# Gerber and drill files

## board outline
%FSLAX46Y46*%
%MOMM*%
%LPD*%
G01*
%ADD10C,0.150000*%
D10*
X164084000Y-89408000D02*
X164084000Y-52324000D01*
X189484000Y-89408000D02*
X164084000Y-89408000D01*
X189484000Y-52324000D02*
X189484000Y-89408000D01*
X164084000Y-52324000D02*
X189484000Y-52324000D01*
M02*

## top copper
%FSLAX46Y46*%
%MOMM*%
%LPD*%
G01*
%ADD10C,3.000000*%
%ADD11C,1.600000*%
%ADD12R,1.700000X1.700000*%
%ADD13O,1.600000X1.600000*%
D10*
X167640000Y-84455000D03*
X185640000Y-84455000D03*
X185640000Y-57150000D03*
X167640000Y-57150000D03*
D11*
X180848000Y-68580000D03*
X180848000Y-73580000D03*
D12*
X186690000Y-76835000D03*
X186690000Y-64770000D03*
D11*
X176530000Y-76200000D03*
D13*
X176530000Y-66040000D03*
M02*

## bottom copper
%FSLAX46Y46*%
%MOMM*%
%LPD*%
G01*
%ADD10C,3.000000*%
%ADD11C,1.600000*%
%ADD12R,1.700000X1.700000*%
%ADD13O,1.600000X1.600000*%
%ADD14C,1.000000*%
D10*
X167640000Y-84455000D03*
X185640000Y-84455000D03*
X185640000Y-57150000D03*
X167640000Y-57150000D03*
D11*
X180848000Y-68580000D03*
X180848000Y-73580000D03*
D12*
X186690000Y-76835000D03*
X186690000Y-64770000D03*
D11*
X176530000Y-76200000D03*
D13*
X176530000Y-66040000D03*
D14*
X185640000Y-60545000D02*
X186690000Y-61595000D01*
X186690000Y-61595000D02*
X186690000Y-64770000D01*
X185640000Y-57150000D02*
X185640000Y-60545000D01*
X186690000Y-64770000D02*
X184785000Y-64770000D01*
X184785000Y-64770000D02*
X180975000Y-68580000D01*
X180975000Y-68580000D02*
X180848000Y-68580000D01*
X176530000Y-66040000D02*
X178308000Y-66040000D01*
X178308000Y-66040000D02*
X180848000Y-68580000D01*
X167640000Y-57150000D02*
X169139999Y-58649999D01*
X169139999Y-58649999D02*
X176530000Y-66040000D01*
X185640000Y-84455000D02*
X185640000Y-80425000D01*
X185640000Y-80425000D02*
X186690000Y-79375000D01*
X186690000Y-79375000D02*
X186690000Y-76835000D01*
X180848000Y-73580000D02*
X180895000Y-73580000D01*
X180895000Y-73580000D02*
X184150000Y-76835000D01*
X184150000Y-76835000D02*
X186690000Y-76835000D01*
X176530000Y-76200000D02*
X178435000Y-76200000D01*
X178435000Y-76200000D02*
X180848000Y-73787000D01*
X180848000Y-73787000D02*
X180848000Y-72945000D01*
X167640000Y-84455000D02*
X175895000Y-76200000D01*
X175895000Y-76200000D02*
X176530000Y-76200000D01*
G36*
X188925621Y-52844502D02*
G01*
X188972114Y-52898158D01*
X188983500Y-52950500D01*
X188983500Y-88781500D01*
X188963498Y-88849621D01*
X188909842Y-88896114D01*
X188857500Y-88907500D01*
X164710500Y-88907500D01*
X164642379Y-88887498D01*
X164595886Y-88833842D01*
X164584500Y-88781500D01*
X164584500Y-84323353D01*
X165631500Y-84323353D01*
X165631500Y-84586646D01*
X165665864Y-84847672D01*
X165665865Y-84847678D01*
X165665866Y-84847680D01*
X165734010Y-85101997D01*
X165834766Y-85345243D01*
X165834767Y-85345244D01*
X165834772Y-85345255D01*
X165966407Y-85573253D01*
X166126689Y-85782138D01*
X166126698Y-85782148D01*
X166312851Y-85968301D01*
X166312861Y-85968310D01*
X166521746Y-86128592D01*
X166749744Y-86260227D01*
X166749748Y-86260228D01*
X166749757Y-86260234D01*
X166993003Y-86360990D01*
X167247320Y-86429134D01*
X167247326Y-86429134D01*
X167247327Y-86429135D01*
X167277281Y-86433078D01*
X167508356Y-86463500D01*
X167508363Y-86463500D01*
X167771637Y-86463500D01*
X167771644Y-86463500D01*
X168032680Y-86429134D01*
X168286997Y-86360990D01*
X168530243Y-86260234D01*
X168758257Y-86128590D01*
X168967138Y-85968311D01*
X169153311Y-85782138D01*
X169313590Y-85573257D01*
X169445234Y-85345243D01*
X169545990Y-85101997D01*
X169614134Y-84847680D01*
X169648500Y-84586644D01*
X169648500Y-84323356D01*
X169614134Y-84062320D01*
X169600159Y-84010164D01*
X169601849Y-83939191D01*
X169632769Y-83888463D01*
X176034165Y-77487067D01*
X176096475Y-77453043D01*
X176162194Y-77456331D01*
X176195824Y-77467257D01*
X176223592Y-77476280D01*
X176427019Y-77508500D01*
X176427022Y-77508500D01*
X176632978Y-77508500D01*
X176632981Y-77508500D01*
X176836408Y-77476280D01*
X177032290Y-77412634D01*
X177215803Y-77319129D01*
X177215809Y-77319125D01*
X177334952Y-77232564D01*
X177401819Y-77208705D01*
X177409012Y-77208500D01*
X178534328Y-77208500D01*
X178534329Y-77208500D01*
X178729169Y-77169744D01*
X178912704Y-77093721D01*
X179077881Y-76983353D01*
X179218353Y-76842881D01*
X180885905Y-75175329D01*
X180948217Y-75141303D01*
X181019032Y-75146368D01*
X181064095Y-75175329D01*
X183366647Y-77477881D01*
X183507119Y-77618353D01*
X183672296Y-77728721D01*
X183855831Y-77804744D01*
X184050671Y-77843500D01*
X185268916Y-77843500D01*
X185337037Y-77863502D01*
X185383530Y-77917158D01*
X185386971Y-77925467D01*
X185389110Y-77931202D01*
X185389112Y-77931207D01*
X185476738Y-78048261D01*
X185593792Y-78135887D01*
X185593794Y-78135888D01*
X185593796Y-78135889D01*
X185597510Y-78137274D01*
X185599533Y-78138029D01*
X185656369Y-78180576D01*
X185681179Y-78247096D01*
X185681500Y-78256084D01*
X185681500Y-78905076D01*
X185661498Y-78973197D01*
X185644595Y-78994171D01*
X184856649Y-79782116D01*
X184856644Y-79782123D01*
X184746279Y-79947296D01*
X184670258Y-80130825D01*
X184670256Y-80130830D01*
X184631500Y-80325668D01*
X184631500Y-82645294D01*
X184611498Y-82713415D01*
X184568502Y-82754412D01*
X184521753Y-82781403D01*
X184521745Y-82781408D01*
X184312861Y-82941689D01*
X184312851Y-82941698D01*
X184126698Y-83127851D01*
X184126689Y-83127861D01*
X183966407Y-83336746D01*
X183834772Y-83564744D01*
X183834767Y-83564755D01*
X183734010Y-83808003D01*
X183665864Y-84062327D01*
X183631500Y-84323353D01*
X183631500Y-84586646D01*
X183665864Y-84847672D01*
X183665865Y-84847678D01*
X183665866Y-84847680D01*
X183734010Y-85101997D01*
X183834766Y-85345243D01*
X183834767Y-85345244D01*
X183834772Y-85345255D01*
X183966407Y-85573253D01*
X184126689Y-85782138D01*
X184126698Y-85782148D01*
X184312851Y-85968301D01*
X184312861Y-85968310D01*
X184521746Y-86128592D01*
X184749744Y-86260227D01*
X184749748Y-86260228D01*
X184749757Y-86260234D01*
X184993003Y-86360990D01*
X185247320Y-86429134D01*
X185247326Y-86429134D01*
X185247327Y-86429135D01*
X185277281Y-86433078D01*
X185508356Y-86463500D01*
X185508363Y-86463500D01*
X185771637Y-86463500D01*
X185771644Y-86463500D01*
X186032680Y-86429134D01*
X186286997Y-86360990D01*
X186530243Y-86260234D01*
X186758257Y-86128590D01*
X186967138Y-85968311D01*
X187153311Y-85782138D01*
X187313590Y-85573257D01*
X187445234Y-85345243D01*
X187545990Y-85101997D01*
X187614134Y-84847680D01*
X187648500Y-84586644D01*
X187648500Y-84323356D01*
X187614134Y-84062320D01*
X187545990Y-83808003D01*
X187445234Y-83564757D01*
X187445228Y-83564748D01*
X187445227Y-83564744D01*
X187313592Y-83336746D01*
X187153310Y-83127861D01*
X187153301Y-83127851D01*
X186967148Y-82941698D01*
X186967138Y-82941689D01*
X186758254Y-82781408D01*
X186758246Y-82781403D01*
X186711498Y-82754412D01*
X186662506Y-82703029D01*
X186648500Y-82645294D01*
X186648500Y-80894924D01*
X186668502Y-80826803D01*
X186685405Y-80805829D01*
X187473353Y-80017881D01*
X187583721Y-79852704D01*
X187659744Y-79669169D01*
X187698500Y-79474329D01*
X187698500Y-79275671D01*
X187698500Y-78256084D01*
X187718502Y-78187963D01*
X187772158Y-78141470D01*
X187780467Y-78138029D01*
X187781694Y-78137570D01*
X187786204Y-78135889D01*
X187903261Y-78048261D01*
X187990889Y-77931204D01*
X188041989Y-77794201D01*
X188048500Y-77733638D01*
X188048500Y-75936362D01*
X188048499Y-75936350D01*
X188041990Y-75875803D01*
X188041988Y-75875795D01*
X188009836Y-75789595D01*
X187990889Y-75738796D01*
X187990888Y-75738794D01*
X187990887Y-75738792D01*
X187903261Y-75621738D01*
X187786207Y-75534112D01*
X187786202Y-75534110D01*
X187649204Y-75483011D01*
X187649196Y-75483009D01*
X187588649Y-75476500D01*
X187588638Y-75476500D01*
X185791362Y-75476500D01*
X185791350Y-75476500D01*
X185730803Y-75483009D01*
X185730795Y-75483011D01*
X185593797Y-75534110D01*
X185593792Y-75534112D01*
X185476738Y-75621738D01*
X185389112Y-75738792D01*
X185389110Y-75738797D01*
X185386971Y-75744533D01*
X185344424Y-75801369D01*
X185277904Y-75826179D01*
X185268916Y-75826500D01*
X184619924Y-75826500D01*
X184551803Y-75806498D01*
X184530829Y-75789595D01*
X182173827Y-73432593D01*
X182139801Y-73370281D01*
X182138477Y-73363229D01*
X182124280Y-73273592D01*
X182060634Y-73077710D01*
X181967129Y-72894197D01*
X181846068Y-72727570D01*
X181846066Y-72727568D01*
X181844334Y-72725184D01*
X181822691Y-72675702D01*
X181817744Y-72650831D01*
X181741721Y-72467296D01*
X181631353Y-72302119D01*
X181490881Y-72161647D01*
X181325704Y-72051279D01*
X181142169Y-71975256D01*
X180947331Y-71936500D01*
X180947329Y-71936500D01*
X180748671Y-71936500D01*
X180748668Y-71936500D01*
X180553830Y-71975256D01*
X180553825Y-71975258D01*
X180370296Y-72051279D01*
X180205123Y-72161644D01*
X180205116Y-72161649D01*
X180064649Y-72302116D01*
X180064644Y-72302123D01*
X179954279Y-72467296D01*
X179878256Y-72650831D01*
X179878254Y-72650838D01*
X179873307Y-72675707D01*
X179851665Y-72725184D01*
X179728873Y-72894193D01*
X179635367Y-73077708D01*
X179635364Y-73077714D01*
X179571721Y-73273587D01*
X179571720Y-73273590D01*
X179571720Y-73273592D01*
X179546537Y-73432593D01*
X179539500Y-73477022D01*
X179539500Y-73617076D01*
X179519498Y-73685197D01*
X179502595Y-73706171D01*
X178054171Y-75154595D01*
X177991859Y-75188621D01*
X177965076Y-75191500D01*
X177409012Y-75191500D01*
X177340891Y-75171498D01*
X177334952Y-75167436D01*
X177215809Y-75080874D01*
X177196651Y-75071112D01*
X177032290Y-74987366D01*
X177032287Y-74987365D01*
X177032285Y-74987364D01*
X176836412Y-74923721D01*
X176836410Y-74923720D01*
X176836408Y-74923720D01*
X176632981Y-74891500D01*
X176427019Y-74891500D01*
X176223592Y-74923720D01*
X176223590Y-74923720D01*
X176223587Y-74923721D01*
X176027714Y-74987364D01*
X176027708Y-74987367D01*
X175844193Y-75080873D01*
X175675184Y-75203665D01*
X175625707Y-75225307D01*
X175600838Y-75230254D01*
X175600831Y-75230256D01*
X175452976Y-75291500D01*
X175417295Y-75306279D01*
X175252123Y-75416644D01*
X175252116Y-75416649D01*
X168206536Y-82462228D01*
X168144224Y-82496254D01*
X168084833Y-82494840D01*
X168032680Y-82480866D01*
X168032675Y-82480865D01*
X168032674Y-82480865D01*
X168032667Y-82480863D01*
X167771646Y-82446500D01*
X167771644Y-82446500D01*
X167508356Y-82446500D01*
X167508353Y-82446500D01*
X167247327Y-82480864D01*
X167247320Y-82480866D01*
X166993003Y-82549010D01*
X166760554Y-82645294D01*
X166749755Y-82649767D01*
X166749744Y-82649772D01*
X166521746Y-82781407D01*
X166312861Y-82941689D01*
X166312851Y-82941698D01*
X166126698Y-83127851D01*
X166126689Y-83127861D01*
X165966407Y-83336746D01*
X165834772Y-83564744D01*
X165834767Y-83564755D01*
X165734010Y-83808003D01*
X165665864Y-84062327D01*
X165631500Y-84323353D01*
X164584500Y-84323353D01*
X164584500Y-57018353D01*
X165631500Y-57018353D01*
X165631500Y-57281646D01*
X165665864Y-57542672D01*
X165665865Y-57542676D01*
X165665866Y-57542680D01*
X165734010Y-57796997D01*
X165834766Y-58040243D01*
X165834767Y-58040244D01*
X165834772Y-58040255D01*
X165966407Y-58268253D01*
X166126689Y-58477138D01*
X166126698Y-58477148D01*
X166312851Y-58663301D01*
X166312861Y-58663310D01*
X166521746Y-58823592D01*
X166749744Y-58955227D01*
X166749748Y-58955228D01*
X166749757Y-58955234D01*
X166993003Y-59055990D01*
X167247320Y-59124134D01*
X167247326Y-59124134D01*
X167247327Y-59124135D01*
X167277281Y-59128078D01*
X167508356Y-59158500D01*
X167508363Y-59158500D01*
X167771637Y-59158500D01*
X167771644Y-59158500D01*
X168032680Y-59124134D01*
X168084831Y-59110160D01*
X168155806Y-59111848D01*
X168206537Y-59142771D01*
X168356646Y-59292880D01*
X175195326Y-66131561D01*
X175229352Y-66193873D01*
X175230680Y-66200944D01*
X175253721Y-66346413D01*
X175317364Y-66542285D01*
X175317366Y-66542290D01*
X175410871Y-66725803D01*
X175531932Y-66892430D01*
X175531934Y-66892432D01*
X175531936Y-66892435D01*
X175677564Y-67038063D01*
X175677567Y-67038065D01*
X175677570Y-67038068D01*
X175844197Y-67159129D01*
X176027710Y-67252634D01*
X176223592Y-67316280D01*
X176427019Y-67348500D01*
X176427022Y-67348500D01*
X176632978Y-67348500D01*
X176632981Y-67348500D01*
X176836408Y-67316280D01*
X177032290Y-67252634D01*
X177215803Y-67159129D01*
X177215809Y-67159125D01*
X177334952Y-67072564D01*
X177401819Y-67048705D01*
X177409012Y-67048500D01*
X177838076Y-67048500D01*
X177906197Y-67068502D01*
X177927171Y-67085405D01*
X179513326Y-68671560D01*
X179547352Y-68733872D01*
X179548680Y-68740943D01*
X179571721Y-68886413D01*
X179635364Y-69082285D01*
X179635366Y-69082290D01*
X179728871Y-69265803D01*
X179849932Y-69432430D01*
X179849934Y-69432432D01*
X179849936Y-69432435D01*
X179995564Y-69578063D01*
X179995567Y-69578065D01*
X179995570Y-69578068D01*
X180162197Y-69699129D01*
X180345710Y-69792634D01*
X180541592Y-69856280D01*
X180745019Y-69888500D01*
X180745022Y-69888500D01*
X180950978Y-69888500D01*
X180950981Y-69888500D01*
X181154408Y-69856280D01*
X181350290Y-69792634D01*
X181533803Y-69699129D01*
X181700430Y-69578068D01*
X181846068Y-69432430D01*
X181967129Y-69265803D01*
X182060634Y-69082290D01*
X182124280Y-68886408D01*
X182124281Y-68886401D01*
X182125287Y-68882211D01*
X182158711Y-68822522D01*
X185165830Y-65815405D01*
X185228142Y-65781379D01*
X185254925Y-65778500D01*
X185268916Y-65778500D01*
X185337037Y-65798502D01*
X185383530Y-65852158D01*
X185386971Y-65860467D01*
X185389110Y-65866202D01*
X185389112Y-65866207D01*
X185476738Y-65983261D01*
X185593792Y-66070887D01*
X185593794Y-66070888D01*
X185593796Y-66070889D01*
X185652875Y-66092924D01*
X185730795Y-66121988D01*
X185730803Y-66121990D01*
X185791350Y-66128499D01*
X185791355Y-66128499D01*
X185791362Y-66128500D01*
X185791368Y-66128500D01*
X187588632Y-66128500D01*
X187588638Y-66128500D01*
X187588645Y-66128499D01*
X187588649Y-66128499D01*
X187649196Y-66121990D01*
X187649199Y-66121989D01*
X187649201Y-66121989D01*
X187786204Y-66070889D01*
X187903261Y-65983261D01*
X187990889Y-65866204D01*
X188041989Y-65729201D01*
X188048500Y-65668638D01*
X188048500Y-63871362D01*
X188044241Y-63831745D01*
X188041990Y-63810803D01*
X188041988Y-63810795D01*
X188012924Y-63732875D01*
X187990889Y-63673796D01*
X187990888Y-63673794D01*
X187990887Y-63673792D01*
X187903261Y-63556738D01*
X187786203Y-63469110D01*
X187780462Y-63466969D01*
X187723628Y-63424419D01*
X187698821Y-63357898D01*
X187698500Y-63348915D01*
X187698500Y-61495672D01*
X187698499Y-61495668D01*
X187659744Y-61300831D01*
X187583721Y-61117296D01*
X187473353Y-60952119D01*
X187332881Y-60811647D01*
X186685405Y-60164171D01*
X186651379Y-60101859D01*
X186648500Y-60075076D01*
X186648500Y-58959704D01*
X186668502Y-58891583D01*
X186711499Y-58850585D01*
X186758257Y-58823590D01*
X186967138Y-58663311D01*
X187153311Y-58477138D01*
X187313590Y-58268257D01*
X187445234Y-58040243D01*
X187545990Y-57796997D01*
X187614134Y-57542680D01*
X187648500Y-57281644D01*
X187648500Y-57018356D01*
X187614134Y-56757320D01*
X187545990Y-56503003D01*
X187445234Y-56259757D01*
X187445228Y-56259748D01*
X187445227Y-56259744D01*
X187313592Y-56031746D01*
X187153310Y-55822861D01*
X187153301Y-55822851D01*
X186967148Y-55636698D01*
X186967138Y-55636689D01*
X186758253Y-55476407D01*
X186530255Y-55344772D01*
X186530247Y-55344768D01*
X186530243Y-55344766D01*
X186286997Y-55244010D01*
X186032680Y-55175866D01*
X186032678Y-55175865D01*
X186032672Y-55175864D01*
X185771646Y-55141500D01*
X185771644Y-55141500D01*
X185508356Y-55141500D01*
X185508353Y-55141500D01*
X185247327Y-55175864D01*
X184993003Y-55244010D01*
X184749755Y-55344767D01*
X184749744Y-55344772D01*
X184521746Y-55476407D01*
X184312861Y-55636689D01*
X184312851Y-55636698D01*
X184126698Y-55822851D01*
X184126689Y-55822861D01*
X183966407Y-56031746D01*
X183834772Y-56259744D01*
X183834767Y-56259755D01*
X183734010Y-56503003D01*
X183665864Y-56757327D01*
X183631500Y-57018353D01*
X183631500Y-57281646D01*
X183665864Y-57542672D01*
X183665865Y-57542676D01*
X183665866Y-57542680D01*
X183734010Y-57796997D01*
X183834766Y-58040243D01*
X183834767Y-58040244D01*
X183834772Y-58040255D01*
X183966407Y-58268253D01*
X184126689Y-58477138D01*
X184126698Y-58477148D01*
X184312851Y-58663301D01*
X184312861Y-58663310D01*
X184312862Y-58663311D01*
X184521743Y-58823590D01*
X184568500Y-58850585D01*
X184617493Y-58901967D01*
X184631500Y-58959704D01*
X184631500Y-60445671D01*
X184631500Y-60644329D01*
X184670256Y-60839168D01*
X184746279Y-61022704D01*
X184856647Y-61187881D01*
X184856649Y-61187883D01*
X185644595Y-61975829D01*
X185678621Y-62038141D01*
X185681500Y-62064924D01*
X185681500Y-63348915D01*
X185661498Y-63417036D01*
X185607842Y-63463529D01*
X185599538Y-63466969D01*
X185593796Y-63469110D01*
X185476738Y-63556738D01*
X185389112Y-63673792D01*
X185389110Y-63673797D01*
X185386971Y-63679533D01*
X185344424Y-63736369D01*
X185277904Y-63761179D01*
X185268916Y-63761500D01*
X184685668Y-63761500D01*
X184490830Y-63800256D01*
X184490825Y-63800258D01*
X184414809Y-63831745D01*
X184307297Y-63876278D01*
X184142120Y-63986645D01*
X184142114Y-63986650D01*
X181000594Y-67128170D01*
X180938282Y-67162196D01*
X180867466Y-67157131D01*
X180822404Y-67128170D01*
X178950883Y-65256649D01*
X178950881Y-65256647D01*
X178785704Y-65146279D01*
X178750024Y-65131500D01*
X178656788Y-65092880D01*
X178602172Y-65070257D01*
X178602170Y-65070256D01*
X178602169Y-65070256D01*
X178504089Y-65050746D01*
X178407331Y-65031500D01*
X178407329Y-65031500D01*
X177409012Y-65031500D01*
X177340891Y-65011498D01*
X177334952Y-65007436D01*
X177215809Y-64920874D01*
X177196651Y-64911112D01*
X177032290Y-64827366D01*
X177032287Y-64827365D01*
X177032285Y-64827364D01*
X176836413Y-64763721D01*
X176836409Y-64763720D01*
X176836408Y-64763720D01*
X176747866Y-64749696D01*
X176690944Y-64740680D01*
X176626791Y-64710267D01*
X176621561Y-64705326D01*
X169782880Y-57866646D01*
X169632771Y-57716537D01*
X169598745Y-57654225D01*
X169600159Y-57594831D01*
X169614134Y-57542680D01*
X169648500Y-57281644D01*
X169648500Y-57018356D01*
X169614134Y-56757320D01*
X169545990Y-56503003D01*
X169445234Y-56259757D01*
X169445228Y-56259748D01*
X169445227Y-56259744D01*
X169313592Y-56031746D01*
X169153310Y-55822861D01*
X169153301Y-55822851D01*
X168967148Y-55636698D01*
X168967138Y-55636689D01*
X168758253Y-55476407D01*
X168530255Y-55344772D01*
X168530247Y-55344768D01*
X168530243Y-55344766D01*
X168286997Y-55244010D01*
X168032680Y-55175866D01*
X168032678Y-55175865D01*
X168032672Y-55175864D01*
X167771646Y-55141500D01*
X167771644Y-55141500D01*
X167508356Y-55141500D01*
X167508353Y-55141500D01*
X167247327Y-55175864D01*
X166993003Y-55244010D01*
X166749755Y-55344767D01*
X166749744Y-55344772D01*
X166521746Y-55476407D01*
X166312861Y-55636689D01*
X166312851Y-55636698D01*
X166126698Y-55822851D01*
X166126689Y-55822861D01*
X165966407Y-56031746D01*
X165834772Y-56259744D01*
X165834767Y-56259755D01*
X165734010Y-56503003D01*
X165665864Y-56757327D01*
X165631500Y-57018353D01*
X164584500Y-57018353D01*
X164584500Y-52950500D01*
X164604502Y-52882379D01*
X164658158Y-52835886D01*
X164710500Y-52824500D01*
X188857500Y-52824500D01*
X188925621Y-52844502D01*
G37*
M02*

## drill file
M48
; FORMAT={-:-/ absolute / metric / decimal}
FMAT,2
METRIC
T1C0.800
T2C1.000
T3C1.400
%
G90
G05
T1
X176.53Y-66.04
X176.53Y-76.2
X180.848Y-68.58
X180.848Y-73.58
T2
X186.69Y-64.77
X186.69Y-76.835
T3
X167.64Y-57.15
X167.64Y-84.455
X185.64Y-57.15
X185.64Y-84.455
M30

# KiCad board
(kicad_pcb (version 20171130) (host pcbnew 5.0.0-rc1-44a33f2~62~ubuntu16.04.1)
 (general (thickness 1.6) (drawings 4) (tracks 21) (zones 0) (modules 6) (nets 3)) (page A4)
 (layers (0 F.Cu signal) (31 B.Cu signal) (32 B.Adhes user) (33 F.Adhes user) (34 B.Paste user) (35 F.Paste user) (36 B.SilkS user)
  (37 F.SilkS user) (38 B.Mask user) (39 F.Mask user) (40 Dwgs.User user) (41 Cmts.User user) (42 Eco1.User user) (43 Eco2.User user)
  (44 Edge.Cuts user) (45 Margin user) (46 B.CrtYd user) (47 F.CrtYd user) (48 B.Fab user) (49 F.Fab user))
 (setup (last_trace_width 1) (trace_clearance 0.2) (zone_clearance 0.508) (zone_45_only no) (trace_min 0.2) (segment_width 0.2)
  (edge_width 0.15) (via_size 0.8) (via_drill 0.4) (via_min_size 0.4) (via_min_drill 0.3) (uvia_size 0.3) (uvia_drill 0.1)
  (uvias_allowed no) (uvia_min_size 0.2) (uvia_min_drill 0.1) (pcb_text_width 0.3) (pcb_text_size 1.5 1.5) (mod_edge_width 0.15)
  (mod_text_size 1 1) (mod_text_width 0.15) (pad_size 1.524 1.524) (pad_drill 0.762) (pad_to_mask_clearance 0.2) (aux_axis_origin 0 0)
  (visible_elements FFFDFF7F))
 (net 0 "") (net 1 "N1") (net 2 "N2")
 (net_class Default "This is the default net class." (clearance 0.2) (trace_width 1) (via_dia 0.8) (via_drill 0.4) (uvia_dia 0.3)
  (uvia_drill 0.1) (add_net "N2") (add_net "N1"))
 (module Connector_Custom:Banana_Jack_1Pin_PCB (layer F.Cu) (at 167.64 84.455 90)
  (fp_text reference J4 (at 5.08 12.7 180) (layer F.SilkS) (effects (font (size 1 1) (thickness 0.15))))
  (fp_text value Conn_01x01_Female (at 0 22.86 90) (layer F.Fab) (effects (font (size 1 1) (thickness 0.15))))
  (pad 1 thru_hole circle (at 0 0 90) (size 3 3) (drill 1.4) (layers *.Cu *.Mask) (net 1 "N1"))
  (pad 1 thru_hole circle (at 0 18 90) (size 3 3) (drill 1.4) (layers *.Cu *.Mask) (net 1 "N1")))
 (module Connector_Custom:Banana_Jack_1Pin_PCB (layer F.Cu) (at 167.64 57.15 90)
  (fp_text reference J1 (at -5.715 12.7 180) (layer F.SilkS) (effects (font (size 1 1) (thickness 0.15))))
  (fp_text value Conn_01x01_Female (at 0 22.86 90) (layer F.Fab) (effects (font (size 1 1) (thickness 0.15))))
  (pad 1 thru_hole circle (at 0 18 90) (size 3 3) (drill 1.4) (layers *.Cu *.Mask) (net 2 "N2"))
  (pad 1 thru_hole circle (at 0 0 90) (size 3 3) (drill 1.4) (layers *.Cu *.Mask) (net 2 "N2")))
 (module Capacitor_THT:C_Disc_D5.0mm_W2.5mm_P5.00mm (layer F.Cu) (at 180.848 68.58 270)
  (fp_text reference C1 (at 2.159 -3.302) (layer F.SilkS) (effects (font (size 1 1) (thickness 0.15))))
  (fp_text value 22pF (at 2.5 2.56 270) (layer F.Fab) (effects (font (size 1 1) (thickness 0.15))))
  (pad 1 thru_hole circle (at 0 0 270) (size 1.6 1.6) (drill 0.8) (layers *.Cu *.Mask) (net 2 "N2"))
  (pad 2 thru_hole circle (at 5 0 270) (size 1.6 1.6) (drill 0.8) (layers *.Cu *.Mask) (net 1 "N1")))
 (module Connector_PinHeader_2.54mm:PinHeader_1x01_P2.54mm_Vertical (layer F.Cu) (at 186.69 76.835)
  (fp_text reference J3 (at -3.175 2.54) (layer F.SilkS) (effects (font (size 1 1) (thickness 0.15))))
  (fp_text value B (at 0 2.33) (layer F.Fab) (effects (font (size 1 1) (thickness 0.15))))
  (pad 1 thru_hole rect (at 0 0) (size 1.7 1.7) (drill 1) (layers *.Cu *.Mask) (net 1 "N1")))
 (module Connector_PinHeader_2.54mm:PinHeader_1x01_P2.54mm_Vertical (layer F.Cu) (at 186.69 64.77)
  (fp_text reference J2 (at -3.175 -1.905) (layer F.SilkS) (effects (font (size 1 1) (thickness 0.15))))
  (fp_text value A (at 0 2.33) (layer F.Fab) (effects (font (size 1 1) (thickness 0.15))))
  (pad 1 thru_hole rect (at 0 0) (size 1.7 1.7) (drill 1) (layers *.Cu *.Mask) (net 2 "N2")))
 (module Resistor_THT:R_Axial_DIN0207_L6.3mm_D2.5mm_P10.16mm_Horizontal (layer F.Cu) (at 176.53 76.2 90)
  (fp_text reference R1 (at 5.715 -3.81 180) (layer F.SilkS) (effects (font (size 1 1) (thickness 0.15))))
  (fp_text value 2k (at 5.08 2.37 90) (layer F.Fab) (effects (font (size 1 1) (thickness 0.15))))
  (pad 1 thru_hole circle (at 0 0 90) (size 1.6 1.6) (drill 0.8) (layers *.Cu *.Mask) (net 1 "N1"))
  (pad 2 thru_hole oval (at 10.16 0 90) (size 1.6 1.6) (drill 0.8) (layers *.Cu *.Mask) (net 2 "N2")))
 (gr_line (start 164.084 89.408) (end 164.084 52.324) (layer Edge.Cuts) (width 0.15))
 (gr_line (start 189.484 89.408) (end 164.084 89.408) (layer Edge.Cuts) (width 0.15))
 (gr_line (start 189.484 52.324) (end 189.484 89.408) (layer Edge.Cuts) (width 0.15))
 (gr_line (start 164.084 52.324) (end 189.484 52.324) (layer Edge.Cuts) (width 0.15))
 (segment (start 185.64 60.545) (end 186.69 61.595) (width 1) (layer B.Cu) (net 2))
 (segment (start 186.69 61.595) (end 186.69 64.77) (width 1) (layer B.Cu) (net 2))
 (segment (start 185.64 57.15) (end 185.64 60.545) (width 1) (layer B.Cu) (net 2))
 (segment (start 186.69 64.77) (end 184.785 64.77) (width 1) (layer B.Cu) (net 2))
 (segment (start 184.785 64.77) (end 180.975 68.58) (width 1) (layer B.Cu) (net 2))
 (segment (start 180.975 68.58) (end 180.848 68.58) (width 1) (layer B.Cu) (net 2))
 (segment (start 176.53 66.04) (end 178.308 66.04) (width 1) (layer B.Cu) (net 2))
 (segment (start 178.308 66.04) (end 180.848 68.58) (width 1) (layer B.Cu) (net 2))
 (segment (start 167.64 57.15) (end 169.139999 58.649999) (width 1) (layer B.Cu) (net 2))
 (segment (start 169.139999 58.649999) (end 176.53 66.04) (width 1) (layer B.Cu) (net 2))
 (segment (start 185.64 84.455) (end 185.64 80.425) (width 1) (layer B.Cu) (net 1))
 (segment (start 185.64 80.425) (end 186.69 79.375) (width 1) (layer B.Cu) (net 1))
 (segment (start 186.69 79.375) (end 186.69 76.835) (width 1) (layer B.Cu) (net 1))
 (segment (start 180.848 73.58) (end 180.895 73.58) (width 1) (layer B.Cu) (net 1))
 (segment (start 180.895 73.58) (end 184.15 76.835) (width 1) (layer B.Cu) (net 1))
 (segment (start 184.15 76.835) (end 186.69 76.835) (width 1) (layer B.Cu) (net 1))
 (segment (start 176.53 76.2) (end 178.435 76.2) (width 1) (layer B.Cu) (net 1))
 (segment (start 178.435 76.2) (end 180.848 73.787) (width 1) (layer B.Cu) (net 1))
 (segment (start 180.848 73.787) (end 180.848 72.945) (width 1) (layer B.Cu) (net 1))
 (segment (start 167.64 84.455) (end 175.895 76.2) (width 1) (layer B.Cu) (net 1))
 (segment (start 175.895 76.2) (end 176.53 76.2) (width 1) (layer B.Cu) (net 1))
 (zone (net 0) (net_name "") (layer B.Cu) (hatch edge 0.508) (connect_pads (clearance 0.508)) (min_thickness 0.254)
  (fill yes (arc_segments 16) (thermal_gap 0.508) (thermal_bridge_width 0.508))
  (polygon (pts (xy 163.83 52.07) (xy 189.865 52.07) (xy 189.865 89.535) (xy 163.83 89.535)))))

